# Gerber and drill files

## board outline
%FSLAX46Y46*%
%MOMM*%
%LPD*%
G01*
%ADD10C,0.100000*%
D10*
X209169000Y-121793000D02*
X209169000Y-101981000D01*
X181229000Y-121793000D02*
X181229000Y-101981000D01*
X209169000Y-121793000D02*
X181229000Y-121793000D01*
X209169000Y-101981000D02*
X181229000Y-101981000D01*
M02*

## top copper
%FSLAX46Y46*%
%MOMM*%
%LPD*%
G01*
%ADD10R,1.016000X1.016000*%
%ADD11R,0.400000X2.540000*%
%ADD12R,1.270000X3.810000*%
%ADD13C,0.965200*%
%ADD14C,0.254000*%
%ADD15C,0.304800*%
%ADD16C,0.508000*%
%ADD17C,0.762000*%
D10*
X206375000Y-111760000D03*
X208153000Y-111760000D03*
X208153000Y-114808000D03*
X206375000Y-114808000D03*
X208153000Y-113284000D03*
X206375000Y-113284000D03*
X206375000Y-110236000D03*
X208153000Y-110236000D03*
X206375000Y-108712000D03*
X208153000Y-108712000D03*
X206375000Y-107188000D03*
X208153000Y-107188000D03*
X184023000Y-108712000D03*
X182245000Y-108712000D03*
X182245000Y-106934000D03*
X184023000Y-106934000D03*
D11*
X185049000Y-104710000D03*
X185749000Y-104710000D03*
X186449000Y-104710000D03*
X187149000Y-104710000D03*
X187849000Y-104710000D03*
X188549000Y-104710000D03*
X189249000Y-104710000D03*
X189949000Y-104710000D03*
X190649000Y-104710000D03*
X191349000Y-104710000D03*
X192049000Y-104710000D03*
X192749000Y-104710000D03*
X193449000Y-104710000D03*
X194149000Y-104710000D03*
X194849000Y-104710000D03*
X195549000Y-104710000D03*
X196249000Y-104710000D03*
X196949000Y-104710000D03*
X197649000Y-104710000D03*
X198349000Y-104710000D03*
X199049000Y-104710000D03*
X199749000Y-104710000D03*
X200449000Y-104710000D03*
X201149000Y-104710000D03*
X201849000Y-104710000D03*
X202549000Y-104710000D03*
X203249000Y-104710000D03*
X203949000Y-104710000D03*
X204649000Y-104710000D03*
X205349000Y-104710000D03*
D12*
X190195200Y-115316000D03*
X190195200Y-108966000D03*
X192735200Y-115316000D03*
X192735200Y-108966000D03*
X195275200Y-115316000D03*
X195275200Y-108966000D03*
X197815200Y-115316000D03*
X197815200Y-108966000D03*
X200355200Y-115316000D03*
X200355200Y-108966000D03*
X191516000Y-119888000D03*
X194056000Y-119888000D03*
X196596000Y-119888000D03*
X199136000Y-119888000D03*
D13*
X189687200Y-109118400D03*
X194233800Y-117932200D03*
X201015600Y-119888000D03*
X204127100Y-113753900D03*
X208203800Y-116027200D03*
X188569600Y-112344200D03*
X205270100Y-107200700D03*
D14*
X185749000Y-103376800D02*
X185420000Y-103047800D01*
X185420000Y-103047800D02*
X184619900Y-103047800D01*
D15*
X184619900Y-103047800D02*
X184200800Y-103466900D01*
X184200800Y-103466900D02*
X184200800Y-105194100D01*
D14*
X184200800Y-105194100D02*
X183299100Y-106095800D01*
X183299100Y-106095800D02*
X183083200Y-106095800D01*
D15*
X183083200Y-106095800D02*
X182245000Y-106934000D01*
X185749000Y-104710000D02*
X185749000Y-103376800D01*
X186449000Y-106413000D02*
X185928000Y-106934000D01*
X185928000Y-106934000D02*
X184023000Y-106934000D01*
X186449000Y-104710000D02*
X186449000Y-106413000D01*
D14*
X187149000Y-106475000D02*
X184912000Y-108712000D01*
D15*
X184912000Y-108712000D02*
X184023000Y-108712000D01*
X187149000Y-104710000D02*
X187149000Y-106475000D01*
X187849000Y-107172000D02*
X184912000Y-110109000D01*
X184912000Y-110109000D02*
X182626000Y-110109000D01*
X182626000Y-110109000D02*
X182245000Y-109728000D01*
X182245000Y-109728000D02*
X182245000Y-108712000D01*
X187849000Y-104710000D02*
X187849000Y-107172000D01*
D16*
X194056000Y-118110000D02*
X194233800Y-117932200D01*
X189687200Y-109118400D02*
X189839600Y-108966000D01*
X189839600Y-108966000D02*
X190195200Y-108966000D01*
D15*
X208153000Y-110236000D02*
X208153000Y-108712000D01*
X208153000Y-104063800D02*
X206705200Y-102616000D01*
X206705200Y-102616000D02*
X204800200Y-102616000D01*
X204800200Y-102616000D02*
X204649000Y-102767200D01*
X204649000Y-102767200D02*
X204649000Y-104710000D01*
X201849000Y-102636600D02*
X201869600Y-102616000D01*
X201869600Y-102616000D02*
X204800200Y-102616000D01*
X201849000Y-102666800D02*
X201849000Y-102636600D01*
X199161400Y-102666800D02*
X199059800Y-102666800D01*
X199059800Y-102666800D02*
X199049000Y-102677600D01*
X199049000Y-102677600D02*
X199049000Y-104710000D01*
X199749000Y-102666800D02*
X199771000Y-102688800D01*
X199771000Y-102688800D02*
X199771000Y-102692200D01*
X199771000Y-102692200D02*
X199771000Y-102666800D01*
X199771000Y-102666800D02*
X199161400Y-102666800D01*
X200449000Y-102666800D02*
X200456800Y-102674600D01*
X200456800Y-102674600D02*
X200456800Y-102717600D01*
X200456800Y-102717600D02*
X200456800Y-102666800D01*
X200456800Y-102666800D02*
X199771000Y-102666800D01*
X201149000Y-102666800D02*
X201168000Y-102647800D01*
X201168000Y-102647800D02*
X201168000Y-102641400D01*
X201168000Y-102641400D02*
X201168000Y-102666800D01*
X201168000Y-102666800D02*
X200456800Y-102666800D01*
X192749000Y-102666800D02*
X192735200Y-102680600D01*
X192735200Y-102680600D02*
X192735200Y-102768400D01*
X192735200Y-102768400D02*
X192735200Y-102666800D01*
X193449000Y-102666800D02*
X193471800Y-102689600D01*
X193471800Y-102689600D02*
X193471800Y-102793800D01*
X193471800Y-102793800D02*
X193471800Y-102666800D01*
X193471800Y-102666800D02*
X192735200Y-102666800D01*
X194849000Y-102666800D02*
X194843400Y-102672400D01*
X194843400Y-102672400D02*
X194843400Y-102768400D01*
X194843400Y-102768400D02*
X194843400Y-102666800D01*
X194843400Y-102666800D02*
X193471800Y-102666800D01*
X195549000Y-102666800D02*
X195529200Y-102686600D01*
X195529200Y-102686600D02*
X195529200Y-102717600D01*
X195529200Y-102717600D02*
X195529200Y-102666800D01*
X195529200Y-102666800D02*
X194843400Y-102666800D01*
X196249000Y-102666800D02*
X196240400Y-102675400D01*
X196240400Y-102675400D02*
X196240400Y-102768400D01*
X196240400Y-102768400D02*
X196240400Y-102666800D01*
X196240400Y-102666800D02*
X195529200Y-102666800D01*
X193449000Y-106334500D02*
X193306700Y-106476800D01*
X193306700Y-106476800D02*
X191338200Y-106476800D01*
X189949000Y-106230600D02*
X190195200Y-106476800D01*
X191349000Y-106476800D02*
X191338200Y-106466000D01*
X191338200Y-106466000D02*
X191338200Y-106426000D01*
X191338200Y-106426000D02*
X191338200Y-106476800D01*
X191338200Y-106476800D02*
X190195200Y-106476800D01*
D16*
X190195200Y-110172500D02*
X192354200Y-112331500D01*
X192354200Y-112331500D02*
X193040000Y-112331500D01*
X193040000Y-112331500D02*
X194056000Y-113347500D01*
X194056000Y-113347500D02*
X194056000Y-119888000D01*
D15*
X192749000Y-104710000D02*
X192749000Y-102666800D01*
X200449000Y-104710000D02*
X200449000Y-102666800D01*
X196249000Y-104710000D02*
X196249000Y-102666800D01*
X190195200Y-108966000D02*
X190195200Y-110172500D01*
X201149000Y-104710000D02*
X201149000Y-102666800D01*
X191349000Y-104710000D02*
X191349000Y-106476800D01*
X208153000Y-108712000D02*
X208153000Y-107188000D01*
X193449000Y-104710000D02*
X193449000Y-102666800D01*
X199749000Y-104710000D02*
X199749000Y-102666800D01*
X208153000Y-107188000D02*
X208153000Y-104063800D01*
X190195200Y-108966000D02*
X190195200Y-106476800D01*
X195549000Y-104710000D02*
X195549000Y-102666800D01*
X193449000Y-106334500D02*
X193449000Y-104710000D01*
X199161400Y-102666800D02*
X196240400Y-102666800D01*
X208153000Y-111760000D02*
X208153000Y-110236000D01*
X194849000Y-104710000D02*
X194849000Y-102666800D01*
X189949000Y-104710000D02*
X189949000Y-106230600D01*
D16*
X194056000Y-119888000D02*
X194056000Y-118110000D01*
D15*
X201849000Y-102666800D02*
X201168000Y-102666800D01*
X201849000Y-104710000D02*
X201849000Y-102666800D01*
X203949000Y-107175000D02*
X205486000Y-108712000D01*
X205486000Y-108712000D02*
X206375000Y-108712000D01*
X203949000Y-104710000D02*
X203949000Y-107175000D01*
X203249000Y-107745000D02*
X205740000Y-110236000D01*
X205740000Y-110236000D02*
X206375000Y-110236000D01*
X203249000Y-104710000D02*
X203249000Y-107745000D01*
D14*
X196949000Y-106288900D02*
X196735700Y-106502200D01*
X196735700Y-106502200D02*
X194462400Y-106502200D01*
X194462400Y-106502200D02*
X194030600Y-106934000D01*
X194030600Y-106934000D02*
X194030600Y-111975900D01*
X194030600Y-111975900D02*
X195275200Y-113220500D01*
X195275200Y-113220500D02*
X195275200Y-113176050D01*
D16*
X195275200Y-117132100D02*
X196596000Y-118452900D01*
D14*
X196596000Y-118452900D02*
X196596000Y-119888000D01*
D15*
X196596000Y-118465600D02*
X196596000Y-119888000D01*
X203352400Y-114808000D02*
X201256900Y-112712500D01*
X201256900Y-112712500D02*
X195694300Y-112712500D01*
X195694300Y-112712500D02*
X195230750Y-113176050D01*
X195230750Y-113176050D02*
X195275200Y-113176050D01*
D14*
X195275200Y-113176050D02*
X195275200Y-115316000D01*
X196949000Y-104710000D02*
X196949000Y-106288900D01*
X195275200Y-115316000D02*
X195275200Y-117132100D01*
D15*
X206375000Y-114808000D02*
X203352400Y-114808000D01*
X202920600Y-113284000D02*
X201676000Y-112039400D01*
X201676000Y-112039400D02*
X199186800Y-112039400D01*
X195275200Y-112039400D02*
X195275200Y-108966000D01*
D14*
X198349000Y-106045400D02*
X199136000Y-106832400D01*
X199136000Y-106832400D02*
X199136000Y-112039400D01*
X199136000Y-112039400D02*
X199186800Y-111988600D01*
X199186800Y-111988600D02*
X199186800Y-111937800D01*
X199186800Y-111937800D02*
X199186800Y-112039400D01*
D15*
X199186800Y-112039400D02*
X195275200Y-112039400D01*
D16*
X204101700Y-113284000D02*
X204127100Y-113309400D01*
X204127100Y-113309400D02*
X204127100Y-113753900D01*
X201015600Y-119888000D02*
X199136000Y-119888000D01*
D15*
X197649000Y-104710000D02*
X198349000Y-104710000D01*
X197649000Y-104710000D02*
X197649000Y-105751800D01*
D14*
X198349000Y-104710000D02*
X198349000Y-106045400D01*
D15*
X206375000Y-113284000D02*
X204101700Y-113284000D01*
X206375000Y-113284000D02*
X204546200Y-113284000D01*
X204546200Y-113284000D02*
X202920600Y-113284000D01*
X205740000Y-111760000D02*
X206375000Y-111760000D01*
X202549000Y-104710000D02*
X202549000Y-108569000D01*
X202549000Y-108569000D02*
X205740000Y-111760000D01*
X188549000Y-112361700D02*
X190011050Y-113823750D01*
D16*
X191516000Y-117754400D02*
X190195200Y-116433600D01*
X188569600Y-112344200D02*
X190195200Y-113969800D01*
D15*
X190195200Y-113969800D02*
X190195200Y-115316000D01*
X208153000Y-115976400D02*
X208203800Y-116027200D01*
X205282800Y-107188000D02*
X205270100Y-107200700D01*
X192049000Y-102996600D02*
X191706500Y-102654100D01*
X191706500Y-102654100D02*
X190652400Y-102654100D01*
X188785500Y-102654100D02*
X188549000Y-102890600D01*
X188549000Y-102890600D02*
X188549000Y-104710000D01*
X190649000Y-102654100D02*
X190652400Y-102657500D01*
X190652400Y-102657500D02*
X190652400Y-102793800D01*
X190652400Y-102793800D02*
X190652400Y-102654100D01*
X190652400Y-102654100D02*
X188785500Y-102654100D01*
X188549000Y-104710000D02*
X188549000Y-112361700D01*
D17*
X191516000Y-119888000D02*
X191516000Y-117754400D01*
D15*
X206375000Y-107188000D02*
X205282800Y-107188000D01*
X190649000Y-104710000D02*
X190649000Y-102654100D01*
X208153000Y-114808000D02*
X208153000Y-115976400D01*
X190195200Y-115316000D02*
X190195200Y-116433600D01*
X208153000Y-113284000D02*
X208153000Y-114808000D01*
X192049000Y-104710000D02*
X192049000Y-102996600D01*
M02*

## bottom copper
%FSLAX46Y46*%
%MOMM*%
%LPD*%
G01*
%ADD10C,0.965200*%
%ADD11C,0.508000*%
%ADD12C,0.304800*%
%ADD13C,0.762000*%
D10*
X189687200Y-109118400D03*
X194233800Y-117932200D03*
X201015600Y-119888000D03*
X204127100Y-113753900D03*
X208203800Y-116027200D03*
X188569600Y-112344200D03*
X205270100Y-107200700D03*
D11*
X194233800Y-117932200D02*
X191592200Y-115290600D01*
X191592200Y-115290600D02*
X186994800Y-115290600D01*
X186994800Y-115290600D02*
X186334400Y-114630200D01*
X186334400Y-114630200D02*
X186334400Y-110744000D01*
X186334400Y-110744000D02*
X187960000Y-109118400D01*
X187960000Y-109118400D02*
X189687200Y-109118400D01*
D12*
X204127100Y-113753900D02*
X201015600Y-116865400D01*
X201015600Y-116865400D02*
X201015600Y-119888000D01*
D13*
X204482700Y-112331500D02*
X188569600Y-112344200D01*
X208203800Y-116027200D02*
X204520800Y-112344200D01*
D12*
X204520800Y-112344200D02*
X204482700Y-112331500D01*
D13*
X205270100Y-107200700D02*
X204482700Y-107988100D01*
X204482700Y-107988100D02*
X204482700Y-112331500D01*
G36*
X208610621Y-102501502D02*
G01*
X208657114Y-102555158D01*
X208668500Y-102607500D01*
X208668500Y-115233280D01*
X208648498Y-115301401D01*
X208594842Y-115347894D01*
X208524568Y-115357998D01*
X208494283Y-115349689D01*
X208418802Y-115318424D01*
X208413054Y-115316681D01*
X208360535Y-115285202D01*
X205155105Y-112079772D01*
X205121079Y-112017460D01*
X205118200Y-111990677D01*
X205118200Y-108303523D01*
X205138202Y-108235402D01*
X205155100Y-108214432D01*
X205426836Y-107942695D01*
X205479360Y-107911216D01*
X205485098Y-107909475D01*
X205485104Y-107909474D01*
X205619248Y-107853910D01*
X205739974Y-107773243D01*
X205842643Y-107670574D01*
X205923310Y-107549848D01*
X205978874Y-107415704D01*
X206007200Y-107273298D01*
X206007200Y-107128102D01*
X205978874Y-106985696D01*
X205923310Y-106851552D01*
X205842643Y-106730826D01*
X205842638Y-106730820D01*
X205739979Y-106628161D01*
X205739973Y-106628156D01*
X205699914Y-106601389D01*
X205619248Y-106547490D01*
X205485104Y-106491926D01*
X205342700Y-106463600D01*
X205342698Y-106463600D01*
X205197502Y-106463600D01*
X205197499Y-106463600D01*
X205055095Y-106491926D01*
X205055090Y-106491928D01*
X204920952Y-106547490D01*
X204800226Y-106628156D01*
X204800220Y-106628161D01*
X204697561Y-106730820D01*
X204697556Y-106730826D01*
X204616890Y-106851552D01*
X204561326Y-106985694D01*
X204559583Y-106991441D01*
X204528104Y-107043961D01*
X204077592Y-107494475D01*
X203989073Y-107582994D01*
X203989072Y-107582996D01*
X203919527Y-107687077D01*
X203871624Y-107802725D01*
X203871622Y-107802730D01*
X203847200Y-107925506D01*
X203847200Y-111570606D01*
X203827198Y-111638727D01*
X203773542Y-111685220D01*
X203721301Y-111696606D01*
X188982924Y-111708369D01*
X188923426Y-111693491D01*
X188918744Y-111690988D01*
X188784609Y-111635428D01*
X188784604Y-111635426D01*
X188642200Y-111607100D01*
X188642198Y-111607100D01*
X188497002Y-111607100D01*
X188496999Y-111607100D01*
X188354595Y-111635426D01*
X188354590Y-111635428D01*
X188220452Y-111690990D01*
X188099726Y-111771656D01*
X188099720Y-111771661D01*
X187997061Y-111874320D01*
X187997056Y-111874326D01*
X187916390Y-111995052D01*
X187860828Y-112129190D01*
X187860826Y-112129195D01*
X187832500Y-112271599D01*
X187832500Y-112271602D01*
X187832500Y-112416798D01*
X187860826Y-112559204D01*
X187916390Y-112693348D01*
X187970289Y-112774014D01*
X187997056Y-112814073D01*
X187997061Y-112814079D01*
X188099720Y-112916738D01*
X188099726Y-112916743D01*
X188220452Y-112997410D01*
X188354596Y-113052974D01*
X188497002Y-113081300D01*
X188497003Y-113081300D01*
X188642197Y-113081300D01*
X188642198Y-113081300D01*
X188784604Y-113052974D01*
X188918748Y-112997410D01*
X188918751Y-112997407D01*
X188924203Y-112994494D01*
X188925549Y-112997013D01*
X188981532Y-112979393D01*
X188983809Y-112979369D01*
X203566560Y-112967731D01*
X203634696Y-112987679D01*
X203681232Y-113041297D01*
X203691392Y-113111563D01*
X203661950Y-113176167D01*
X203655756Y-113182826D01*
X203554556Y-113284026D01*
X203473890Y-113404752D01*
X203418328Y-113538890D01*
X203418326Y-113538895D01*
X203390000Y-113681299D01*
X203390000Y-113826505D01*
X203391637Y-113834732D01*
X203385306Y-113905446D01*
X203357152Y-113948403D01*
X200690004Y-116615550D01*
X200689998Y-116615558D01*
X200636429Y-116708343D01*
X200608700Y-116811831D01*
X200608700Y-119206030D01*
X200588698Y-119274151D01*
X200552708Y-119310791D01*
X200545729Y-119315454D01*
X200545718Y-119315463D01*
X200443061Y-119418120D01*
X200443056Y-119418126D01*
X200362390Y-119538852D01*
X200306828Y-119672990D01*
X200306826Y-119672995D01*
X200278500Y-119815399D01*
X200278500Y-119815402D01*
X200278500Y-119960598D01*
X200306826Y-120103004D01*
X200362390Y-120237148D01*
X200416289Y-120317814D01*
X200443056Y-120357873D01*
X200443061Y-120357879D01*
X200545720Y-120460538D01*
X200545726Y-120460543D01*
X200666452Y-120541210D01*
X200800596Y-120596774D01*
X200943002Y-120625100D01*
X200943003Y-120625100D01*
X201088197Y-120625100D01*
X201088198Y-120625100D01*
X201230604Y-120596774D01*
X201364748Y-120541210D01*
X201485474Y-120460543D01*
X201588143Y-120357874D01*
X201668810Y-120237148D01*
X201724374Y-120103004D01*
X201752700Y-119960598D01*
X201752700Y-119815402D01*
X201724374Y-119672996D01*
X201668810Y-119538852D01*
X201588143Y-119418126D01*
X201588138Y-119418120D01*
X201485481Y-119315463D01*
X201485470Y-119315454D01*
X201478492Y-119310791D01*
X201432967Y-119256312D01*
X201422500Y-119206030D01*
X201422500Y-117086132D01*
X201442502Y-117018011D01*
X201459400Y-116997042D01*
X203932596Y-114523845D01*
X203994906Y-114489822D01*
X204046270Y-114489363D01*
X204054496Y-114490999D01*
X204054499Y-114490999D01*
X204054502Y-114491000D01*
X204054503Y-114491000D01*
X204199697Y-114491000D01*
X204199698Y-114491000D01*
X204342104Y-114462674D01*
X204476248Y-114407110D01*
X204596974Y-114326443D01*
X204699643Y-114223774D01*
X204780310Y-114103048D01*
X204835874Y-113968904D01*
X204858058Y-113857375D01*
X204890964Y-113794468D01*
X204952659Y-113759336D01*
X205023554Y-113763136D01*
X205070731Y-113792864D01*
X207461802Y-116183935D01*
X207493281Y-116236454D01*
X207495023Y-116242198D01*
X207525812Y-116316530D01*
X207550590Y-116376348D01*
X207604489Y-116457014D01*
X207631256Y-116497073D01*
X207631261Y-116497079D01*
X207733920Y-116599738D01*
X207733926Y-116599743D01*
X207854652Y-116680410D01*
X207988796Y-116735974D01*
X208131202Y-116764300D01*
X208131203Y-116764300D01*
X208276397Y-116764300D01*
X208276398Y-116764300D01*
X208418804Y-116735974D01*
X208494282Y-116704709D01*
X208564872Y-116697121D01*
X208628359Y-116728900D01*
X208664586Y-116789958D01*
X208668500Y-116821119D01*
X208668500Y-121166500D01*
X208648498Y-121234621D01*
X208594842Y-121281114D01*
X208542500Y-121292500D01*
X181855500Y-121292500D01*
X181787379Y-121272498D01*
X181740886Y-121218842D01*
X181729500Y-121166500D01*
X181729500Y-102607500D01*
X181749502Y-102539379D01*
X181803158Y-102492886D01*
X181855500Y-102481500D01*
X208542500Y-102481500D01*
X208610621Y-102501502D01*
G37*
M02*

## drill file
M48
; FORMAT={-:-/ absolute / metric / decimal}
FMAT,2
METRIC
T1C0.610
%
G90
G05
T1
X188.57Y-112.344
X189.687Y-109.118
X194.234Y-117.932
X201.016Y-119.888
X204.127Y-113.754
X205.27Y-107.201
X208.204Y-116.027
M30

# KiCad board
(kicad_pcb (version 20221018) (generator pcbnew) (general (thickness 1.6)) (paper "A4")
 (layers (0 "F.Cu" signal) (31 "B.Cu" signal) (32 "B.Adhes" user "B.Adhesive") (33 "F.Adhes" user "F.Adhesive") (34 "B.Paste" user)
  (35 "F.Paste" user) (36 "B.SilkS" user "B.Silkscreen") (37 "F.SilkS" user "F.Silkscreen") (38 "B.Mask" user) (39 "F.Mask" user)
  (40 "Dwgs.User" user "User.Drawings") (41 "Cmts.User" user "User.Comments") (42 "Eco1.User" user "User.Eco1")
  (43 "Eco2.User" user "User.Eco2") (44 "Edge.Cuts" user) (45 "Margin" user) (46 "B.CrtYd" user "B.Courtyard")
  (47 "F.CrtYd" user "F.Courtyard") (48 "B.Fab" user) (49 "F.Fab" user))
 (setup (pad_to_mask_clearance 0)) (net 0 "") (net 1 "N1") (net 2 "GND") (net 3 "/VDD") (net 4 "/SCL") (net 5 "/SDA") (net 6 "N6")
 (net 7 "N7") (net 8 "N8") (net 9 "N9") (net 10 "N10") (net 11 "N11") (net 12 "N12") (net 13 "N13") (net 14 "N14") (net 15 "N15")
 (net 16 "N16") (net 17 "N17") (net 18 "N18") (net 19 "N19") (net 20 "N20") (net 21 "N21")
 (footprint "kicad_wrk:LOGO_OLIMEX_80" (layer "F.Cu") (at 205.5876 118.6942)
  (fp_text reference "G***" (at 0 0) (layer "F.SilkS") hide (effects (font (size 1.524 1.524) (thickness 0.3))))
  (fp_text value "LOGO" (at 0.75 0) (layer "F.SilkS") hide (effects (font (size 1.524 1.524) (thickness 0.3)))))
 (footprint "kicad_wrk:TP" (layer "F.Cu") (at 182.753 103.378 180)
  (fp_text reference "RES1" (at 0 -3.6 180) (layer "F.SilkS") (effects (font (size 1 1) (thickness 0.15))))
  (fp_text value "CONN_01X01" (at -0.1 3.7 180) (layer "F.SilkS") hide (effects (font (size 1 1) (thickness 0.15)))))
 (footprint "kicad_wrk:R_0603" (layer "F.Cu") (at 207.264 111.76)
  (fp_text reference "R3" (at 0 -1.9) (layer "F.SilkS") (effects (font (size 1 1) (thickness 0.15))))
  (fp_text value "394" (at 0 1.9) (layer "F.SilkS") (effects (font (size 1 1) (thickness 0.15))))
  (pad "1" smd rect (at -0.889 0) (size 1.016 1.016) (layers "F.Cu" "F.Paste" "F.Mask") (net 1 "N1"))
  (pad "2" smd rect (at 0.889 0) (size 1.016 1.016) (layers "F.Cu" "F.Paste" "F.Mask") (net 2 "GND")))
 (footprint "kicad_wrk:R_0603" (layer "F.Cu") (at 207.264 114.808 180)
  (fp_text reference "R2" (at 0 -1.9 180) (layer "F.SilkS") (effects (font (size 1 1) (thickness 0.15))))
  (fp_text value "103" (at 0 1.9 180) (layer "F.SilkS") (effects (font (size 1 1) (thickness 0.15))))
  (pad "1" smd rect (at -0.889 0 180) (size 1.016 1.016) (layers "F.Cu" "F.Paste" "F.Mask") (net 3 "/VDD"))
  (pad "2" smd rect (at 0.889 0 180) (size 1.016 1.016) (layers "F.Cu" "F.Paste" "F.Mask") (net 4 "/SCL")))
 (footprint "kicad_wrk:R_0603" (layer "F.Cu") (at 207.264 113.284 180)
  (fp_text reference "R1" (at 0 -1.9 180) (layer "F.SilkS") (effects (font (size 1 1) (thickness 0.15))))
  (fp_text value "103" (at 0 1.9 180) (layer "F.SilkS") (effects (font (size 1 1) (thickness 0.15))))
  (pad "1" smd rect (at -0.889 0 180) (size 1.016 1.016) (layers "F.Cu" "F.Paste" "F.Mask") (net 3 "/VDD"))
  (pad "2" smd rect (at 0.889 0 180) (size 1.016 1.016) (layers "F.Cu" "F.Paste" "F.Mask") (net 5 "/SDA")))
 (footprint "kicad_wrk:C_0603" (layer "F.Cu") (at 207.264 110.236)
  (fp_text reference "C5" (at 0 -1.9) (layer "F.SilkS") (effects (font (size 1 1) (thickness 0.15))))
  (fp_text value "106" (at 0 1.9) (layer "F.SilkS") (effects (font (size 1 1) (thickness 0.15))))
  (pad "1" smd rect (at -0.889 0) (size 1.016 1.016) (layers "F.Cu" "F.Paste" "F.Mask") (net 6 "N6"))
  (pad "2" smd rect (at 0.889 0) (size 1.016 1.016) (layers "F.Cu" "F.Paste" "F.Mask") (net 2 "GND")))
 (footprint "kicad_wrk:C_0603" (layer "F.Cu") (at 207.264 108.712)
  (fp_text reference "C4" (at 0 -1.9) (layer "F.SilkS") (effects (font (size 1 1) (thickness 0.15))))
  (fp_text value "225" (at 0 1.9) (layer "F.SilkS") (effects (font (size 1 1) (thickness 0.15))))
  (pad "1" smd rect (at -0.889 0) (size 1.016 1.016) (layers "F.Cu" "F.Paste" "F.Mask") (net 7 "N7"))
  (pad "2" smd rect (at 0.889 0) (size 1.016 1.016) (layers "F.Cu" "F.Paste" "F.Mask") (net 2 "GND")))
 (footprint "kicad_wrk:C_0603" (layer "F.Cu") (at 207.264 107.188)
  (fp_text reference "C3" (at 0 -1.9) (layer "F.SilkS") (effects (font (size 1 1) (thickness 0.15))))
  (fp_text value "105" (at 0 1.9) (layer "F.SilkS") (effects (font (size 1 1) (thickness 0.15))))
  (pad "1" smd rect (at -0.889 0) (size 1.016 1.016) (layers "F.Cu" "F.Paste" "F.Mask") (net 3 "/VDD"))
  (pad "2" smd rect (at 0.889 0) (size 1.016 1.016) (layers "F.Cu" "F.Paste" "F.Mask") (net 2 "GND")))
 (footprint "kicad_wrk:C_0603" (layer "F.Cu") (at 183.134 108.712 180)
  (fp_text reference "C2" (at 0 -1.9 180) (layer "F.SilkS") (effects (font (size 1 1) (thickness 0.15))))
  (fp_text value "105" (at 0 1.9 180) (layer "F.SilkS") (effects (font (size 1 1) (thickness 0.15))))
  (pad "1" smd rect (at -0.889 0 180) (size 1.016 1.016) (layers "F.Cu" "F.Paste" "F.Mask") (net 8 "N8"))
  (pad "2" smd rect (at 0.889 0 180) (size 1.016 1.016) (layers "F.Cu" "F.Paste" "F.Mask") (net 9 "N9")))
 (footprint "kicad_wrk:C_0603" (layer "F.Cu") (at 183.134 106.934)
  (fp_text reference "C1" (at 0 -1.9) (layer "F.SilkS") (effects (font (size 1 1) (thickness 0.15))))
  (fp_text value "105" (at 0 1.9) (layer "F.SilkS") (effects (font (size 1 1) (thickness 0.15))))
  (pad "1" smd rect (at -0.889 0) (size 1.016 1.016) (layers "F.Cu" "F.Paste" "F.Mask") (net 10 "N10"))
  (pad "2" smd rect (at 0.889 0) (size 1.016 1.016) (layers "F.Cu" "F.Paste" "F.Mask") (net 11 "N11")))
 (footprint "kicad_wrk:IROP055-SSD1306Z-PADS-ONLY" (layer "F.Cu") (at 195.199 105.41)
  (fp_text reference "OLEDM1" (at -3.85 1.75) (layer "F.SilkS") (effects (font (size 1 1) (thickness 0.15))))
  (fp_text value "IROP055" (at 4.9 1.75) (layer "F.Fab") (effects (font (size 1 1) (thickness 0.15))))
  (pad "1" smd rect (at -10.15 -0.7) (size 0.4 2.54) (layers "F.Cu" "F.Paste" "F.Mask") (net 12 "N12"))
  (pad "2" smd rect (at -9.45 -0.7) (size 0.4 2.54) (layers "F.Cu" "F.Paste" "F.Mask") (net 10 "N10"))
  (pad "3" smd rect (at -8.75 -0.7) (size 0.4 2.54) (layers "F.Cu" "F.Paste" "F.Mask") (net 11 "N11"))
  (pad "4" smd rect (at -8.05 -0.7) (size 0.4 2.54) (layers "F.Cu" "F.Paste" "F.Mask") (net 8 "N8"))
  (pad "5" smd rect (at -7.35 -0.7) (size 0.4 2.54) (layers "F.Cu" "F.Paste" "F.Mask") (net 9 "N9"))
  (pad "6" smd rect (at -6.65 -0.7) (size 0.4 2.54) (layers "F.Cu" "F.Paste" "F.Mask") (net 3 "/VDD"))
  (pad "7" smd rect (at -5.95 -0.7) (size 0.4 2.54) (layers "F.Cu" "F.Paste" "F.Mask") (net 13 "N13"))
  (pad "8" smd rect (at -5.25 -0.7) (size 0.4 2.54) (layers "F.Cu" "F.Paste" "F.Mask") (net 2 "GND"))
  (pad "9" smd rect (at -4.55 -0.7) (size 0.4 2.54) (layers "F.Cu" "F.Paste" "F.Mask") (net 3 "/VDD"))
  (pad "10" smd rect (at -3.85 -0.7) (size 0.4 2.54) (layers "F.Cu" "F.Paste" "F.Mask") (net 2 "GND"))
  (pad "11" smd rect (at -3.15 -0.7) (size 0.4 2.54) (layers "F.Cu" "F.Paste" "F.Mask") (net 3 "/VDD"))
  (pad "12" smd rect (at -2.45 -0.7) (size 0.4 2.54) (layers "F.Cu" "F.Paste" "F.Mask") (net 2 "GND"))
  (pad "13" smd rect (at -1.75 -0.7) (size 0.4 2.54) (layers "F.Cu" "F.Paste" "F.Mask") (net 2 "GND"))
  (pad "14" smd rect (at -1.05 -0.7) (size 0.4 2.54) (layers "F.Cu" "F.Paste" "F.Mask") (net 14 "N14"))
  (pad "15" smd rect (at -0.35 -0.7) (size 0.4 2.54) (layers "F.Cu" "F.Paste" "F.Mask") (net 2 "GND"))
  (pad "16" smd rect (at 0.35 -0.7) (size 0.4 2.54) (layers "F.Cu" "F.Paste" "F.Mask") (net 2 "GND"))
  (pad "17" smd rect (at 1.05 -0.7) (size 0.4 2.54) (layers "F.Cu" "F.Paste" "F.Mask") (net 2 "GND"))
  (pad "18" smd rect (at 1.75 -0.7) (size 0.4 2.54) (layers "F.Cu" "F.Paste" "F.Mask") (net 4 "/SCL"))
  (pad "19" smd rect (at 2.45 -0.7) (size 0.4 2.54) (layers "F.Cu" "F.Paste" "F.Mask") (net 5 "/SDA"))
  (pad "20" smd rect (at 3.15 -0.7) (size 0.4 2.54) (layers "F.Cu" "F.Paste" "F.Mask") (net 5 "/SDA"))
  (pad "21" smd rect (at 3.85 -0.7) (size 0.4 2.54) (layers "F.Cu" "F.Paste" "F.Mask") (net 2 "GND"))
  (pad "22" smd rect (at 4.55 -0.7) (size 0.4 2.54) (layers "F.Cu" "F.Paste" "F.Mask") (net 2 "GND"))
  (pad "23" smd rect (at 5.25 -0.7) (size 0.4 2.54) (layers "F.Cu" "F.Paste" "F.Mask") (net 2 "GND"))
  (pad "24" smd rect (at 5.95 -0.7) (size 0.4 2.54) (layers "F.Cu" "F.Paste" "F.Mask") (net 2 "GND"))
  (pad "25" smd rect (at 6.65 -0.7) (size 0.4 2.54) (layers "F.Cu" "F.Paste" "F.Mask") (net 2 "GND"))
  (pad "26" smd rect (at 7.35 -0.7) (size 0.4 2.54) (layers "F.Cu" "F.Paste" "F.Mask") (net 1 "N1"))
  (pad "27" smd rect (at 8.05 -0.7) (size 0.4 2.54) (layers "F.Cu" "F.Paste" "F.Mask") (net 6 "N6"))
  (pad "28" smd rect (at 8.75 -0.7) (size 0.4 2.54) (layers "F.Cu" "F.Paste" "F.Mask") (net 7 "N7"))
  (pad "29" smd rect (at 9.45 -0.7) (size 0.4 2.54) (layers "F.Cu" "F.Paste" "F.Mask") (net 2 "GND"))
  (pad "30" smd rect (at 10.15 -0.7) (size 0.4 2.54) (layers "F.Cu" "F.Paste" "F.Mask") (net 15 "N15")))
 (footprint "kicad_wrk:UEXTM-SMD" (layer "F.Cu") (at 195.2752 112.141 180)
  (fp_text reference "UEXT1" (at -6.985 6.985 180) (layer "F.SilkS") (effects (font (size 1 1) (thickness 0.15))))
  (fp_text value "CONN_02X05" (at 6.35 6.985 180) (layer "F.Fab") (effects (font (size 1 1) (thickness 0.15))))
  (pad "1" smd rect (at 5.08 -3.175 180) (size 1.27 3.81) (layers "F.Cu" "F.Paste" "F.Mask") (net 3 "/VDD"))
  (pad "2" smd rect (at 5.08 3.175 180) (size 1.27 3.81) (layers "F.Cu" "F.Paste" "F.Mask") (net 2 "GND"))
  (pad "3" smd rect (at 2.54 -3.175 180) (size 1.27 3.81) (layers "F.Cu" "F.Paste" "F.Mask") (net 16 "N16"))
  (pad "4" smd rect (at 2.54 3.175 180) (size 1.27 3.81) (layers "F.Cu" "F.Paste" "F.Mask") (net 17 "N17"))
  (pad "5" smd rect (at 0 -3.175 180) (size 1.27 3.81) (layers "F.Cu" "F.Paste" "F.Mask") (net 4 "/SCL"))
  (pad "6" smd rect (at 0 3.175 180) (size 1.27 3.81) (layers "F.Cu" "F.Paste" "F.Mask") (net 5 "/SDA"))
  (pad "7" smd rect (at -2.54 -3.175 180) (size 1.27 3.81) (layers "F.Cu" "F.Paste" "F.Mask") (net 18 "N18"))
  (pad "8" smd rect (at -2.54 3.175 180) (size 1.27 3.81) (layers "F.Cu" "F.Paste" "F.Mask") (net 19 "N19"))
  (pad "9" smd rect (at -5.08 -3.175 180) (size 1.27 3.81) (layers "F.Cu" "F.Paste" "F.Mask") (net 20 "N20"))
  (pad "10" smd rect (at -5.08 3.175 180) (size 1.27 3.81) (layers "F.Cu" "F.Paste" "F.Mask") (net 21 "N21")))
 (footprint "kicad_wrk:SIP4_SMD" (layer "F.Cu") (at 195.326 119.888)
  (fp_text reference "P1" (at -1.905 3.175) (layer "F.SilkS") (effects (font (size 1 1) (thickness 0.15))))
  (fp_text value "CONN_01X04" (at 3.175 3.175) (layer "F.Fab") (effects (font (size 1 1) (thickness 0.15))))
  (pad "1" smd rect (at -3.81 0) (size 1.27 3.81) (layers "F.Cu" "F.Mask") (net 3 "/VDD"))
  (pad "2" smd rect (at -1.27 0) (size 1.27 3.81) (layers "F.Cu" "F.Mask") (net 2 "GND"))
  (pad "3" smd rect (at 1.27 0) (size 1.27 3.81) (layers "F.Cu" "F.Mask") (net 4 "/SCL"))
  (pad "4" smd rect (at 3.81 0) (size 1.27 3.81) (layers "F.Cu" "F.Mask") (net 5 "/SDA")))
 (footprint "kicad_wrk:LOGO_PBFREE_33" (layer "F.Cu") (at 183.6166 118.8466)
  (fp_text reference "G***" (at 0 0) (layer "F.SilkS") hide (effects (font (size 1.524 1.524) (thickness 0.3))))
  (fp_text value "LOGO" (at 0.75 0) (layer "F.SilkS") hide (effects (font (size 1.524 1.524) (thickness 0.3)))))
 (gr_line (start 209.169 121.793) (end 209.169 101.981) (stroke (width 0.1) (type solid)) (layer "Edge.Cuts"))
 (gr_line (start 181.229 121.793) (end 181.229 101.981) (stroke (width 0.1) (type solid)) (layer "Edge.Cuts"))
 (gr_line (start 209.169 121.793) (end 181.229 121.793) (stroke (width 0.1) (type solid)) (layer "Edge.Cuts"))
 (gr_line (start 209.169 101.981) (end 181.229 101.981) (stroke (width 0.1) (type solid)) (layer "Edge.Cuts"))
 (segment (start 185.749 103.3768) (end 185.42 103.0478) (width 0.254) (layer "F.Cu") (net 10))
 (segment (start 185.42 103.0478) (end 184.6199 103.0478) (width 0.254) (layer "F.Cu") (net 10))
 (segment (start 184.6199 103.0478) (end 184.2008 103.4669) (width 0.3048) (layer "F.Cu") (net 10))
 (segment (start 184.2008 103.4669) (end 184.2008 105.1941) (width 0.3048) (layer "F.Cu") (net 10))
 (segment (start 184.2008 105.1941) (end 183.2991 106.0958) (width 0.254) (layer "F.Cu") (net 10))
 (segment (start 183.2991 106.0958) (end 183.0832 106.0958) (width 0.254) (layer "F.Cu") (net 10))
 (segment (start 183.0832 106.0958) (end 182.245 106.934) (width 0.3048) (layer "F.Cu") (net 10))
 (segment (start 185.749 104.71) (end 185.749 103.3768) (width 0.3048) (layer "F.Cu") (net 10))
 (segment (start 186.449 106.413) (end 185.928 106.934) (width 0.3048) (layer "F.Cu") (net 11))
 (segment (start 185.928 106.934) (end 184.023 106.934) (width 0.3048) (layer "F.Cu") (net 11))
 (segment (start 186.449 104.71) (end 186.449 106.413) (width 0.3048) (layer "F.Cu") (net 11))
 (segment (start 187.149 106.475) (end 184.912 108.712) (width 0.254) (layer "F.Cu") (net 8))
 (segment (start 184.912 108.712) (end 184.023 108.712) (width 0.3048) (layer "F.Cu") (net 8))
 (segment (start 187.149 104.71) (end 187.149 106.475) (width 0.3048) (layer "F.Cu") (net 8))
 (segment (start 187.849 107.172) (end 184.912 110.109) (width 0.3048) (layer "F.Cu") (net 9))
 (segment (start 184.912 110.109) (end 182.626 110.109) (width 0.3048) (layer "F.Cu") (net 9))
 (segment (start 182.626 110.109) (end 182.245 109.728) (width 0.3048) (layer "F.Cu") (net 9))
 (segment (start 182.245 109.728) (end 182.245 108.712) (width 0.3048) (layer "F.Cu") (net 9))
 (segment (start 187.849 104.71) (end 187.849 107.172) (width 0.3048) (layer "F.Cu") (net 9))
 (segment (start 194.056 118.11) (end 194.2338 117.9322) (width 0.508) (layer "F.Cu") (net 2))
 (segment (start 189.6872 109.1184) (end 189.8396 108.966) (width 0.508) (layer "F.Cu") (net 2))
 (segment (start 189.8396 108.966) (end 190.1952 108.966) (width 0.508) (layer "F.Cu") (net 2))
 (segment (start 208.153 110.236) (end 208.153 108.712) (width 0.3048) (layer "F.Cu") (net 2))
 (segment (start 208.153 104.0638) (end 206.7052 102.616) (width 0.3048) (layer "F.Cu") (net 2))
 (segment (start 206.7052 102.616) (end 204.8002 102.616) (width 0.3048) (layer "F.Cu") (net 2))
 (segment (start 204.8002 102.616) (end 204.649 102.7672) (width 0.3048) (layer "F.Cu") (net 2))
 (segment (start 204.649 102.7672) (end 204.649 104.71) (width 0.3048) (layer "F.Cu") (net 2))
 (segment (start 201.849 102.6366) (end 201.8696 102.616) (width 0.3048) (layer "F.Cu") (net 2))
 (segment (start 201.8696 102.616) (end 204.8002 102.616) (width 0.3048) (layer "F.Cu") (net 2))
 (segment (start 201.849 102.6668) (end 201.849 102.6366) (width 0.3048) (layer "F.Cu") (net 2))
 (segment (start 199.1614 102.6668) (end 199.0598 102.6668) (width 0.3048) (layer "F.Cu") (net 2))
 (segment (start 199.0598 102.6668) (end 199.049 102.6776) (width 0.3048) (layer "F.Cu") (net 2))
 (segment (start 199.049 102.6776) (end 199.049 104.71) (width 0.3048) (layer "F.Cu") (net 2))
 (segment (start 199.749 102.6668) (end 199.771 102.6888) (width 0.3048) (layer "F.Cu") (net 2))
 (segment (start 199.771 102.6888) (end 199.771 102.6922) (width 0.3048) (layer "F.Cu") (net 2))
 (segment (start 199.771 102.6922) (end 199.771 102.6668) (width 0.3048) (layer "F.Cu") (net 2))
 (segment (start 199.771 102.6668) (end 199.1614 102.6668) (width 0.3048) (layer "F.Cu") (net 2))
 (segment (start 200.449 102.6668) (end 200.4568 102.6746) (width 0.3048) (layer "F.Cu") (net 2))
 (segment (start 200.4568 102.6746) (end 200.4568 102.7176) (width 0.3048) (layer "F.Cu") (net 2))
 (segment (start 200.4568 102.7176) (end 200.4568 102.6668) (width 0.3048) (layer "F.Cu") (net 2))
 (segment (start 200.4568 102.6668) (end 199.771 102.6668) (width 0.3048) (layer "F.Cu") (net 2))
 (segment (start 201.149 102.6668) (end 201.168 102.6478) (width 0.3048) (layer "F.Cu") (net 2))
 (segment (start 201.168 102.6478) (end 201.168 102.6414) (width 0.3048) (layer "F.Cu") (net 2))
 (segment (start 201.168 102.6414) (end 201.168 102.6668) (width 0.3048) (layer "F.Cu") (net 2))
 (segment (start 201.168 102.6668) (end 200.4568 102.6668) (width 0.3048) (layer "F.Cu") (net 2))
 (segment (start 192.749 102.6668) (end 192.7352 102.6806) (width 0.3048) (layer "F.Cu") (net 2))
 (segment (start 192.7352 102.6806) (end 192.7352 102.7684) (width 0.3048) (layer "F.Cu") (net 2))
 (segment (start 192.7352 102.7684) (end 192.7352 102.6668) (width 0.3048) (layer "F.Cu") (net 2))
 (segment (start 193.449 102.6668) (end 193.4718 102.6896) (width 0.3048) (layer "F.Cu") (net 2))
 (segment (start 193.4718 102.6896) (end 193.4718 102.7938) (width 0.3048) (layer "F.Cu") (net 2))
 (segment (start 193.4718 102.7938) (end 193.4718 102.6668) (width 0.3048) (layer "F.Cu") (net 2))
 (segment (start 193.4718 102.6668) (end 192.7352 102.6668) (width 0.3048) (layer "F.Cu") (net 2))
 (segment (start 194.849 102.6668) (end 194.8434 102.6724) (width 0.3048) (layer "F.Cu") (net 2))
 (segment (start 194.8434 102.6724) (end 194.8434 102.7684) (width 0.3048) (layer "F.Cu") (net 2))
 (segment (start 194.8434 102.7684) (end 194.8434 102.6668) (width 0.3048) (layer "F.Cu") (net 2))
 (segment (start 194.8434 102.6668) (end 193.4718 102.6668) (width 0.3048) (layer "F.Cu") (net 2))
 (segment (start 195.549 102.6668) (end 195.5292 102.6866) (width 0.3048) (layer "F.Cu") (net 2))
 (segment (start 195.5292 102.6866) (end 195.5292 102.7176) (width 0.3048) (layer "F.Cu") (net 2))
 (segment (start 195.5292 102.7176) (end 195.5292 102.6668) (width 0.3048) (layer "F.Cu") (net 2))
 (segment (start 195.5292 102.6668) (end 194.8434 102.6668) (width 0.3048) (layer "F.Cu") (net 2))
 (segment (start 196.249 102.6668) (end 196.2404 102.6754) (width 0.3048) (layer "F.Cu") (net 2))
 (segment (start 196.2404 102.6754) (end 196.2404 102.7684) (width 0.3048) (layer "F.Cu") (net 2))
 (segment (start 196.2404 102.7684) (end 196.2404 102.6668) (width 0.3048) (layer "F.Cu") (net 2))
 (segment (start 196.2404 102.6668) (end 195.5292 102.6668) (width 0.3048) (layer "F.Cu") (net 2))
 (segment (start 193.449 106.3345) (end 193.3067 106.4768) (width 0.3048) (layer "F.Cu") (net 2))
 (segment (start 193.3067 106.4768) (end 191.3382 106.4768) (width 0.3048) (layer "F.Cu") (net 2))
 (segment (start 189.949 106.2306) (end 190.1952 106.4768) (width 0.3048) (layer "F.Cu") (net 2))
 (segment (start 191.349 106.4768) (end 191.3382 106.466) (width 0.3048) (layer "F.Cu") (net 2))
 (segment (start 191.3382 106.466) (end 191.3382 106.426) (width 0.3048) (layer "F.Cu") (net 2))
 (segment (start 191.3382 106.426) (end 191.3382 106.4768) (width 0.3048) (layer "F.Cu") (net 2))
 (segment (start 191.3382 106.4768) (end 190.1952 106.4768) (width 0.3048) (layer "F.Cu") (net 2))
 (segment (start 190.1952 110.1725) (end 192.3542 112.3315) (width 0.508) (layer "F.Cu") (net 2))
 (segment (start 192.3542 112.3315) (end 193.04 112.3315) (width 0.508) (layer "F.Cu") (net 2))
 (segment (start 193.04 112.3315) (end 194.056 113.3475) (width 0.508) (layer "F.Cu") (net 2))
 (segment (start 194.056 113.3475) (end 194.056 119.888) (width 0.508) (layer "F.Cu") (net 2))
 (segment (start 192.749 104.71) (end 192.749 102.6668) (width 0.3048) (layer "F.Cu") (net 2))
 (segment (start 200.449 104.71) (end 200.449 102.6668) (width 0.3048) (layer "F.Cu") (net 2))
 (segment (start 196.249 104.71) (end 196.249 102.6668) (width 0.3048) (layer "F.Cu") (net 2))
 (segment (start 190.1952 108.966) (end 190.1952 110.1725) (width 0.3048) (layer "F.Cu") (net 2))
 (segment (start 201.149 104.71) (end 201.149 102.6668) (width 0.3048) (layer "F.Cu") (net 2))
 (segment (start 191.349 104.71) (end 191.349 106.4768) (width 0.3048) (layer "F.Cu") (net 2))
 (segment (start 208.153 108.712) (end 208.153 107.188) (width 0.3048) (layer "F.Cu") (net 2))
 (segment (start 193.449 104.71) (end 193.449 102.6668) (width 0.3048) (layer "F.Cu") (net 2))
 (segment (start 199.749 104.71) (end 199.749 102.6668) (width 0.3048) (layer "F.Cu") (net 2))
 (segment (start 208.153 107.188) (end 208.153 104.0638) (width 0.3048) (layer "F.Cu") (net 2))
 (segment (start 190.1952 108.966) (end 190.1952 106.4768) (width 0.3048) (layer "F.Cu") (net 2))
 (segment (start 195.549 104.71) (end 195.549 102.6668) (width 0.3048) (layer "F.Cu") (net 2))
 (segment (start 193.449 106.3345) (end 193.449 104.71) (width 0.3048) (layer "F.Cu") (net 2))
 (segment (start 199.1614 102.6668) (end 196.2404 102.6668) (width 0.3048) (layer "F.Cu") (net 2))
 (segment (start 208.153 111.76) (end 208.153 110.236) (width 0.3048) (layer "F.Cu") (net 2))
 (segment (start 194.849 104.71) (end 194.849 102.6668) (width 0.3048) (layer "F.Cu") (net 2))
 (segment (start 189.949 104.71) (end 189.949 106.2306) (width 0.3048) (layer "F.Cu") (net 2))
 (segment (start 194.056 119.888) (end 194.056 118.11) (width 0.508) (layer "F.Cu") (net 2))
 (segment (start 201.849 102.6668) (end 201.168 102.6668) (width 0.3048) (layer "F.Cu") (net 2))
 (segment (start 201.849 104.71) (end 201.849 102.6668) (width 0.3048) (layer "F.Cu") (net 2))
 (via (at 189.6872 109.1184) (size 0.9652) (drill 0.6096) (layers "F.Cu" "B.Cu") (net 2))
 (via (at 194.2338 117.9322) (size 0.9652) (drill 0.6096) (layers "F.Cu" "B.Cu") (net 2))
 (segment (start 194.2338 117.9322) (end 191.5922 115.2906) (width 0.508) (layer "B.Cu") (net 2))
 (segment (start 191.5922 115.2906) (end 186.9948 115.2906) (width 0.508) (layer "B.Cu") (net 2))
 (segment (start 186.9948 115.2906) (end 186.3344 114.6302) (width 0.508) (layer "B.Cu") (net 2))
 (segment (start 186.3344 114.6302) (end 186.3344 110.744) (width 0.508) (layer "B.Cu") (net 2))
 (segment (start 186.3344 110.744) (end 187.96 109.1184) (width 0.508) (layer "B.Cu") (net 2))
 (segment (start 187.96 109.1184) (end 189.6872 109.1184) (width 0.508) (layer "B.Cu") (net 2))
 (segment (start 203.949 107.175) (end 205.486 108.712) (width 0.3048) (layer "F.Cu") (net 7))
 (segment (start 205.486 108.712) (end 206.375 108.712) (width 0.3048) (layer "F.Cu") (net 7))
 (segment (start 203.949 104.71) (end 203.949 107.175) (width 0.3048) (layer "F.Cu") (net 7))
 (segment (start 203.249 107.745) (end 205.74 110.236) (width 0.3048) (layer "F.Cu") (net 6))
 (segment (start 205.74 110.236) (end 206.375 110.236) (width 0.3048) (layer "F.Cu") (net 6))
 (segment (start 203.249 104.71) (end 203.249 107.745) (width 0.3048) (layer "F.Cu") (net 6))
 (segment (start 196.949 106.2889) (end 196.7357 106.5022) (width 0.254) (layer "F.Cu") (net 4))
 (segment (start 196.7357 106.5022) (end 194.4624 106.5022) (width 0.254) (layer "F.Cu") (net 4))
 (segment (start 194.4624 106.5022) (end 194.0306 106.934) (width 0.254) (layer "F.Cu") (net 4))
 (segment (start 194.0306 106.934) (end 194.0306 111.9759) (width 0.254) (layer "F.Cu") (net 4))
 (segment (start 194.0306 111.9759) (end 195.2752 113.2205) (width 0.254) (layer "F.Cu") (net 4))
 (segment (start 195.2752 113.2205) (end 195.2752 113.17605) (width 0.254) (layer "F.Cu") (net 4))
 (segment (start 195.2752 117.1321) (end 196.596 118.4529) (width 0.508) (layer "F.Cu") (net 4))
 (segment (start 196.596 118.4529) (end 196.596 119.888) (width 0.254) (layer "F.Cu") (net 4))
 (segment (start 196.596 118.4656) (end 196.596 119.888) (width 0.3048) (layer "F.Cu") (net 4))
 (segment (start 203.3524 114.808) (end 201.2569 112.7125) (width 0.3048) (layer "F.Cu") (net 4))
 (segment (start 201.2569 112.7125) (end 195.6943 112.7125) (width 0.3048) (layer "F.Cu") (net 4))
 (segment (start 195.6943 112.7125) (end 195.23075 113.17605) (width 0.3048) (layer "F.Cu") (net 4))
 (segment (start 195.23075 113.17605) (end 195.2752 113.17605) (width 0.3048) (layer "F.Cu") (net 4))
 (segment (start 195.2752 113.17605) (end 195.2752 115.316) (width 0.254) (layer "F.Cu") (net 4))
 (segment (start 196.949 104.71) (end 196.949 106.2889) (width 0.254) (layer "F.Cu") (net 4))
 (segment (start 195.2752 115.316) (end 195.2752 117.1321) (width 0.254) (layer "F.Cu") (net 4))
 (segment (start 206.375 114.808) (end 203.3524 114.808) (width 0.3048) (layer "F.Cu") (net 4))
 (segment (start 202.9206 113.284) (end 201.676 112.0394) (width 0.3048) (layer "F.Cu") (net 5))
 (segment (start 201.676 112.0394) (end 199.1868 112.0394) (width 0.3048) (layer "F.Cu") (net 5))
 (segment (start 195.2752 112.0394) (end 195.2752 108.966) (width 0.3048) (layer "F.Cu") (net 5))
 (segment (start 198.349 106.0454) (end 199.136 106.8324) (width 0.254) (layer "F.Cu") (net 5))
 (segment (start 199.136 106.8324) (end 199.136 112.0394) (width 0.254) (layer "F.Cu") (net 5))
 (segment (start 199.136 112.0394) (end 199.1868 111.9886) (width 0.254) (layer "F.Cu") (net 5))
 (segment (start 199.1868 111.9886) (end 199.1868 111.9378) (width 0.254) (layer "F.Cu") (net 5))
 (segment (start 199.1868 111.9378) (end 199.1868 112.0394) (width 0.254) (layer "F.Cu") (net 5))
 (segment (start 199.1868 112.0394) (end 195.2752 112.0394) (width 0.3048) (layer "F.Cu") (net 5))
 (segment (start 204.1017 113.284) (end 204.1271 113.3094) (width 0.508) (layer "F.Cu") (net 5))
 (segment (start 204.1271 113.3094) (end 204.1271 113.7539) (width 0.508) (layer "F.Cu") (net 5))
 (segment (start 201.0156 119.888) (end 199.136 119.888) (width 0.508) (layer "F.Cu") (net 5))
 (segment (start 197.649 104.71) (end 198.349 104.71) (width 0.3048) (layer "F.Cu") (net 5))
 (segment (start 197.649 104.71) (end 197.649 105.7518) (width 0.3048) (layer "F.Cu") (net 5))
 (segment (start 198.349 104.71) (end 198.349 106.0454) (width 0.254) (layer "F.Cu") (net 5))
 (segment (start 206.375 113.284) (end 204.1017 113.284) (width 0.3048) (layer "F.Cu") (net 5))
 (segment (start 206.375 113.284) (end 204.5462 113.284) (width 0.3048) (layer "F.Cu") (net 5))
 (segment (start 204.5462 113.284) (end 202.9206 113.284) (width 0.3048) (layer "F.Cu") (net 5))
 (via (at 201.0156 119.888) (size 0.9652) (drill 0.6096) (layers "F.Cu" "B.Cu") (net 5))
 (via (at 204.1271 113.7539) (size 0.9652) (drill 0.6096) (layers "F.Cu" "B.Cu") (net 5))
 (segment (start 204.1271 113.7539) (end 201.0156 116.8654) (width 0.3048) (layer "B.Cu") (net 5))
 (segment (start 201.0156 116.8654) (end 201.0156 119.888) (width 0.3048) (layer "B.Cu") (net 5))
 (segment (start 205.74 111.76) (end 206.375 111.76) (width 0.3048) (layer "F.Cu") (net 1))
 (segment (start 202.549 104.71) (end 202.549 108.569) (width 0.3048) (layer "F.Cu") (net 1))
 (segment (start 202.549 108.569) (end 205.74 111.76) (width 0.3048) (layer "F.Cu") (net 1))
 (segment (start 188.549 112.3617) (end 190.01105 113.82375) (width 0.3048) (layer "F.Cu") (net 3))
 (segment (start 191.516 117.7544) (end 190.1952 116.4336) (width 0.508) (layer "F.Cu") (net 3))
 (segment (start 188.5696 112.3442) (end 190.1952 113.9698) (width 0.508) (layer "F.Cu") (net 3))
 (segment (start 190.1952 113.9698) (end 190.1952 115.316) (width 0.3048) (layer "F.Cu") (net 3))
 (segment (start 208.153 115.9764) (end 208.2038 116.0272) (width 0.3048) (layer "F.Cu") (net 3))
 (segment (start 205.2828 107.188) (end 205.2701 107.2007) (width 0.3048) (layer "F.Cu") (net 3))
 (segment (start 192.049 102.9966) (end 191.7065 102.6541) (width 0.3048) (layer "F.Cu") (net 3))
 (segment (start 191.7065 102.6541) (end 190.6524 102.6541) (width 0.3048) (layer "F.Cu") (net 3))
 (segment (start 188.7855 102.6541) (end 188.549 102.8906) (width 0.3048) (layer "F.Cu") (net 3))
 (segment (start 188.549 102.8906) (end 188.549 104.71) (width 0.3048) (layer "F.Cu") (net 3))
 (segment (start 190.649 102.6541) (end 190.6524 102.6575) (width 0.3048) (layer "F.Cu") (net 3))
 (segment (start 190.6524 102.6575) (end 190.6524 102.7938) (width 0.3048) (layer "F.Cu") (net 3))
 (segment (start 190.6524 102.7938) (end 190.6524 102.6541) (width 0.3048) (layer "F.Cu") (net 3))
 (segment (start 190.6524 102.6541) (end 188.7855 102.6541) (width 0.3048) (layer "F.Cu") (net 3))
 (segment (start 188.549 104.71) (end 188.549 112.3617) (width 0.3048) (layer "F.Cu") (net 3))
 (segment (start 191.516 119.888) (end 191.516 117.7544) (width 0.762) (layer "F.Cu") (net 3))
 (segment (start 206.375 107.188) (end 205.2828 107.188) (width 0.3048) (layer "F.Cu") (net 3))
 (segment (start 190.649 104.71) (end 190.649 102.6541) (width 0.3048) (layer "F.Cu") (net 3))
 (segment (start 208.153 114.808) (end 208.153 115.9764) (width 0.3048) (layer "F.Cu") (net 3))
 (segment (start 190.1952 115.316) (end 190.1952 116.4336) (width 0.3048) (layer "F.Cu") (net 3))
 (segment (start 208.153 113.284) (end 208.153 114.808) (width 0.3048) (layer "F.Cu") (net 3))
 (segment (start 192.049 104.71) (end 192.049 102.9966) (width 0.3048) (layer "F.Cu") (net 3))
 (via (at 208.2038 116.0272) (size 0.9652) (drill 0.6096) (layers "F.Cu" "B.Cu") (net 3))
 (via (at 188.5696 112.3442) (size 0.9652) (drill 0.6096) (layers "F.Cu" "B.Cu") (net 3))
 (via (at 205.2701 107.2007) (size 0.9652) (drill 0.6096) (layers "F.Cu" "B.Cu") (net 3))
 (segment (start 204.4827 112.3315) (end 188.5696 112.3442) (width 0.762) (layer "B.Cu") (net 3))
 (segment (start 208.2038 116.0272) (end 204.5208 112.3442) (width 0.762) (layer "B.Cu") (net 3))
 (segment (start 204.5208 112.3442) (end 204.4827 112.3315) (width 0.3048) (layer "B.Cu") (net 3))
 (segment (start 205.2701 107.2007) (end 204.4827 107.9881) (width 0.762) (layer "B.Cu") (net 3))
 (segment (start 204.4827 107.9881) (end 204.4827 112.3315) (width 0.762) (layer "B.Cu") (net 3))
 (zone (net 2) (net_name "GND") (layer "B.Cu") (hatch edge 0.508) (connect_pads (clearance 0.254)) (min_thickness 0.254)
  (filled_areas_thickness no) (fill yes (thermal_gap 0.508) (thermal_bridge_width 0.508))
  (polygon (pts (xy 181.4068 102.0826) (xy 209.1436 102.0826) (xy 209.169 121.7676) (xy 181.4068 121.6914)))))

